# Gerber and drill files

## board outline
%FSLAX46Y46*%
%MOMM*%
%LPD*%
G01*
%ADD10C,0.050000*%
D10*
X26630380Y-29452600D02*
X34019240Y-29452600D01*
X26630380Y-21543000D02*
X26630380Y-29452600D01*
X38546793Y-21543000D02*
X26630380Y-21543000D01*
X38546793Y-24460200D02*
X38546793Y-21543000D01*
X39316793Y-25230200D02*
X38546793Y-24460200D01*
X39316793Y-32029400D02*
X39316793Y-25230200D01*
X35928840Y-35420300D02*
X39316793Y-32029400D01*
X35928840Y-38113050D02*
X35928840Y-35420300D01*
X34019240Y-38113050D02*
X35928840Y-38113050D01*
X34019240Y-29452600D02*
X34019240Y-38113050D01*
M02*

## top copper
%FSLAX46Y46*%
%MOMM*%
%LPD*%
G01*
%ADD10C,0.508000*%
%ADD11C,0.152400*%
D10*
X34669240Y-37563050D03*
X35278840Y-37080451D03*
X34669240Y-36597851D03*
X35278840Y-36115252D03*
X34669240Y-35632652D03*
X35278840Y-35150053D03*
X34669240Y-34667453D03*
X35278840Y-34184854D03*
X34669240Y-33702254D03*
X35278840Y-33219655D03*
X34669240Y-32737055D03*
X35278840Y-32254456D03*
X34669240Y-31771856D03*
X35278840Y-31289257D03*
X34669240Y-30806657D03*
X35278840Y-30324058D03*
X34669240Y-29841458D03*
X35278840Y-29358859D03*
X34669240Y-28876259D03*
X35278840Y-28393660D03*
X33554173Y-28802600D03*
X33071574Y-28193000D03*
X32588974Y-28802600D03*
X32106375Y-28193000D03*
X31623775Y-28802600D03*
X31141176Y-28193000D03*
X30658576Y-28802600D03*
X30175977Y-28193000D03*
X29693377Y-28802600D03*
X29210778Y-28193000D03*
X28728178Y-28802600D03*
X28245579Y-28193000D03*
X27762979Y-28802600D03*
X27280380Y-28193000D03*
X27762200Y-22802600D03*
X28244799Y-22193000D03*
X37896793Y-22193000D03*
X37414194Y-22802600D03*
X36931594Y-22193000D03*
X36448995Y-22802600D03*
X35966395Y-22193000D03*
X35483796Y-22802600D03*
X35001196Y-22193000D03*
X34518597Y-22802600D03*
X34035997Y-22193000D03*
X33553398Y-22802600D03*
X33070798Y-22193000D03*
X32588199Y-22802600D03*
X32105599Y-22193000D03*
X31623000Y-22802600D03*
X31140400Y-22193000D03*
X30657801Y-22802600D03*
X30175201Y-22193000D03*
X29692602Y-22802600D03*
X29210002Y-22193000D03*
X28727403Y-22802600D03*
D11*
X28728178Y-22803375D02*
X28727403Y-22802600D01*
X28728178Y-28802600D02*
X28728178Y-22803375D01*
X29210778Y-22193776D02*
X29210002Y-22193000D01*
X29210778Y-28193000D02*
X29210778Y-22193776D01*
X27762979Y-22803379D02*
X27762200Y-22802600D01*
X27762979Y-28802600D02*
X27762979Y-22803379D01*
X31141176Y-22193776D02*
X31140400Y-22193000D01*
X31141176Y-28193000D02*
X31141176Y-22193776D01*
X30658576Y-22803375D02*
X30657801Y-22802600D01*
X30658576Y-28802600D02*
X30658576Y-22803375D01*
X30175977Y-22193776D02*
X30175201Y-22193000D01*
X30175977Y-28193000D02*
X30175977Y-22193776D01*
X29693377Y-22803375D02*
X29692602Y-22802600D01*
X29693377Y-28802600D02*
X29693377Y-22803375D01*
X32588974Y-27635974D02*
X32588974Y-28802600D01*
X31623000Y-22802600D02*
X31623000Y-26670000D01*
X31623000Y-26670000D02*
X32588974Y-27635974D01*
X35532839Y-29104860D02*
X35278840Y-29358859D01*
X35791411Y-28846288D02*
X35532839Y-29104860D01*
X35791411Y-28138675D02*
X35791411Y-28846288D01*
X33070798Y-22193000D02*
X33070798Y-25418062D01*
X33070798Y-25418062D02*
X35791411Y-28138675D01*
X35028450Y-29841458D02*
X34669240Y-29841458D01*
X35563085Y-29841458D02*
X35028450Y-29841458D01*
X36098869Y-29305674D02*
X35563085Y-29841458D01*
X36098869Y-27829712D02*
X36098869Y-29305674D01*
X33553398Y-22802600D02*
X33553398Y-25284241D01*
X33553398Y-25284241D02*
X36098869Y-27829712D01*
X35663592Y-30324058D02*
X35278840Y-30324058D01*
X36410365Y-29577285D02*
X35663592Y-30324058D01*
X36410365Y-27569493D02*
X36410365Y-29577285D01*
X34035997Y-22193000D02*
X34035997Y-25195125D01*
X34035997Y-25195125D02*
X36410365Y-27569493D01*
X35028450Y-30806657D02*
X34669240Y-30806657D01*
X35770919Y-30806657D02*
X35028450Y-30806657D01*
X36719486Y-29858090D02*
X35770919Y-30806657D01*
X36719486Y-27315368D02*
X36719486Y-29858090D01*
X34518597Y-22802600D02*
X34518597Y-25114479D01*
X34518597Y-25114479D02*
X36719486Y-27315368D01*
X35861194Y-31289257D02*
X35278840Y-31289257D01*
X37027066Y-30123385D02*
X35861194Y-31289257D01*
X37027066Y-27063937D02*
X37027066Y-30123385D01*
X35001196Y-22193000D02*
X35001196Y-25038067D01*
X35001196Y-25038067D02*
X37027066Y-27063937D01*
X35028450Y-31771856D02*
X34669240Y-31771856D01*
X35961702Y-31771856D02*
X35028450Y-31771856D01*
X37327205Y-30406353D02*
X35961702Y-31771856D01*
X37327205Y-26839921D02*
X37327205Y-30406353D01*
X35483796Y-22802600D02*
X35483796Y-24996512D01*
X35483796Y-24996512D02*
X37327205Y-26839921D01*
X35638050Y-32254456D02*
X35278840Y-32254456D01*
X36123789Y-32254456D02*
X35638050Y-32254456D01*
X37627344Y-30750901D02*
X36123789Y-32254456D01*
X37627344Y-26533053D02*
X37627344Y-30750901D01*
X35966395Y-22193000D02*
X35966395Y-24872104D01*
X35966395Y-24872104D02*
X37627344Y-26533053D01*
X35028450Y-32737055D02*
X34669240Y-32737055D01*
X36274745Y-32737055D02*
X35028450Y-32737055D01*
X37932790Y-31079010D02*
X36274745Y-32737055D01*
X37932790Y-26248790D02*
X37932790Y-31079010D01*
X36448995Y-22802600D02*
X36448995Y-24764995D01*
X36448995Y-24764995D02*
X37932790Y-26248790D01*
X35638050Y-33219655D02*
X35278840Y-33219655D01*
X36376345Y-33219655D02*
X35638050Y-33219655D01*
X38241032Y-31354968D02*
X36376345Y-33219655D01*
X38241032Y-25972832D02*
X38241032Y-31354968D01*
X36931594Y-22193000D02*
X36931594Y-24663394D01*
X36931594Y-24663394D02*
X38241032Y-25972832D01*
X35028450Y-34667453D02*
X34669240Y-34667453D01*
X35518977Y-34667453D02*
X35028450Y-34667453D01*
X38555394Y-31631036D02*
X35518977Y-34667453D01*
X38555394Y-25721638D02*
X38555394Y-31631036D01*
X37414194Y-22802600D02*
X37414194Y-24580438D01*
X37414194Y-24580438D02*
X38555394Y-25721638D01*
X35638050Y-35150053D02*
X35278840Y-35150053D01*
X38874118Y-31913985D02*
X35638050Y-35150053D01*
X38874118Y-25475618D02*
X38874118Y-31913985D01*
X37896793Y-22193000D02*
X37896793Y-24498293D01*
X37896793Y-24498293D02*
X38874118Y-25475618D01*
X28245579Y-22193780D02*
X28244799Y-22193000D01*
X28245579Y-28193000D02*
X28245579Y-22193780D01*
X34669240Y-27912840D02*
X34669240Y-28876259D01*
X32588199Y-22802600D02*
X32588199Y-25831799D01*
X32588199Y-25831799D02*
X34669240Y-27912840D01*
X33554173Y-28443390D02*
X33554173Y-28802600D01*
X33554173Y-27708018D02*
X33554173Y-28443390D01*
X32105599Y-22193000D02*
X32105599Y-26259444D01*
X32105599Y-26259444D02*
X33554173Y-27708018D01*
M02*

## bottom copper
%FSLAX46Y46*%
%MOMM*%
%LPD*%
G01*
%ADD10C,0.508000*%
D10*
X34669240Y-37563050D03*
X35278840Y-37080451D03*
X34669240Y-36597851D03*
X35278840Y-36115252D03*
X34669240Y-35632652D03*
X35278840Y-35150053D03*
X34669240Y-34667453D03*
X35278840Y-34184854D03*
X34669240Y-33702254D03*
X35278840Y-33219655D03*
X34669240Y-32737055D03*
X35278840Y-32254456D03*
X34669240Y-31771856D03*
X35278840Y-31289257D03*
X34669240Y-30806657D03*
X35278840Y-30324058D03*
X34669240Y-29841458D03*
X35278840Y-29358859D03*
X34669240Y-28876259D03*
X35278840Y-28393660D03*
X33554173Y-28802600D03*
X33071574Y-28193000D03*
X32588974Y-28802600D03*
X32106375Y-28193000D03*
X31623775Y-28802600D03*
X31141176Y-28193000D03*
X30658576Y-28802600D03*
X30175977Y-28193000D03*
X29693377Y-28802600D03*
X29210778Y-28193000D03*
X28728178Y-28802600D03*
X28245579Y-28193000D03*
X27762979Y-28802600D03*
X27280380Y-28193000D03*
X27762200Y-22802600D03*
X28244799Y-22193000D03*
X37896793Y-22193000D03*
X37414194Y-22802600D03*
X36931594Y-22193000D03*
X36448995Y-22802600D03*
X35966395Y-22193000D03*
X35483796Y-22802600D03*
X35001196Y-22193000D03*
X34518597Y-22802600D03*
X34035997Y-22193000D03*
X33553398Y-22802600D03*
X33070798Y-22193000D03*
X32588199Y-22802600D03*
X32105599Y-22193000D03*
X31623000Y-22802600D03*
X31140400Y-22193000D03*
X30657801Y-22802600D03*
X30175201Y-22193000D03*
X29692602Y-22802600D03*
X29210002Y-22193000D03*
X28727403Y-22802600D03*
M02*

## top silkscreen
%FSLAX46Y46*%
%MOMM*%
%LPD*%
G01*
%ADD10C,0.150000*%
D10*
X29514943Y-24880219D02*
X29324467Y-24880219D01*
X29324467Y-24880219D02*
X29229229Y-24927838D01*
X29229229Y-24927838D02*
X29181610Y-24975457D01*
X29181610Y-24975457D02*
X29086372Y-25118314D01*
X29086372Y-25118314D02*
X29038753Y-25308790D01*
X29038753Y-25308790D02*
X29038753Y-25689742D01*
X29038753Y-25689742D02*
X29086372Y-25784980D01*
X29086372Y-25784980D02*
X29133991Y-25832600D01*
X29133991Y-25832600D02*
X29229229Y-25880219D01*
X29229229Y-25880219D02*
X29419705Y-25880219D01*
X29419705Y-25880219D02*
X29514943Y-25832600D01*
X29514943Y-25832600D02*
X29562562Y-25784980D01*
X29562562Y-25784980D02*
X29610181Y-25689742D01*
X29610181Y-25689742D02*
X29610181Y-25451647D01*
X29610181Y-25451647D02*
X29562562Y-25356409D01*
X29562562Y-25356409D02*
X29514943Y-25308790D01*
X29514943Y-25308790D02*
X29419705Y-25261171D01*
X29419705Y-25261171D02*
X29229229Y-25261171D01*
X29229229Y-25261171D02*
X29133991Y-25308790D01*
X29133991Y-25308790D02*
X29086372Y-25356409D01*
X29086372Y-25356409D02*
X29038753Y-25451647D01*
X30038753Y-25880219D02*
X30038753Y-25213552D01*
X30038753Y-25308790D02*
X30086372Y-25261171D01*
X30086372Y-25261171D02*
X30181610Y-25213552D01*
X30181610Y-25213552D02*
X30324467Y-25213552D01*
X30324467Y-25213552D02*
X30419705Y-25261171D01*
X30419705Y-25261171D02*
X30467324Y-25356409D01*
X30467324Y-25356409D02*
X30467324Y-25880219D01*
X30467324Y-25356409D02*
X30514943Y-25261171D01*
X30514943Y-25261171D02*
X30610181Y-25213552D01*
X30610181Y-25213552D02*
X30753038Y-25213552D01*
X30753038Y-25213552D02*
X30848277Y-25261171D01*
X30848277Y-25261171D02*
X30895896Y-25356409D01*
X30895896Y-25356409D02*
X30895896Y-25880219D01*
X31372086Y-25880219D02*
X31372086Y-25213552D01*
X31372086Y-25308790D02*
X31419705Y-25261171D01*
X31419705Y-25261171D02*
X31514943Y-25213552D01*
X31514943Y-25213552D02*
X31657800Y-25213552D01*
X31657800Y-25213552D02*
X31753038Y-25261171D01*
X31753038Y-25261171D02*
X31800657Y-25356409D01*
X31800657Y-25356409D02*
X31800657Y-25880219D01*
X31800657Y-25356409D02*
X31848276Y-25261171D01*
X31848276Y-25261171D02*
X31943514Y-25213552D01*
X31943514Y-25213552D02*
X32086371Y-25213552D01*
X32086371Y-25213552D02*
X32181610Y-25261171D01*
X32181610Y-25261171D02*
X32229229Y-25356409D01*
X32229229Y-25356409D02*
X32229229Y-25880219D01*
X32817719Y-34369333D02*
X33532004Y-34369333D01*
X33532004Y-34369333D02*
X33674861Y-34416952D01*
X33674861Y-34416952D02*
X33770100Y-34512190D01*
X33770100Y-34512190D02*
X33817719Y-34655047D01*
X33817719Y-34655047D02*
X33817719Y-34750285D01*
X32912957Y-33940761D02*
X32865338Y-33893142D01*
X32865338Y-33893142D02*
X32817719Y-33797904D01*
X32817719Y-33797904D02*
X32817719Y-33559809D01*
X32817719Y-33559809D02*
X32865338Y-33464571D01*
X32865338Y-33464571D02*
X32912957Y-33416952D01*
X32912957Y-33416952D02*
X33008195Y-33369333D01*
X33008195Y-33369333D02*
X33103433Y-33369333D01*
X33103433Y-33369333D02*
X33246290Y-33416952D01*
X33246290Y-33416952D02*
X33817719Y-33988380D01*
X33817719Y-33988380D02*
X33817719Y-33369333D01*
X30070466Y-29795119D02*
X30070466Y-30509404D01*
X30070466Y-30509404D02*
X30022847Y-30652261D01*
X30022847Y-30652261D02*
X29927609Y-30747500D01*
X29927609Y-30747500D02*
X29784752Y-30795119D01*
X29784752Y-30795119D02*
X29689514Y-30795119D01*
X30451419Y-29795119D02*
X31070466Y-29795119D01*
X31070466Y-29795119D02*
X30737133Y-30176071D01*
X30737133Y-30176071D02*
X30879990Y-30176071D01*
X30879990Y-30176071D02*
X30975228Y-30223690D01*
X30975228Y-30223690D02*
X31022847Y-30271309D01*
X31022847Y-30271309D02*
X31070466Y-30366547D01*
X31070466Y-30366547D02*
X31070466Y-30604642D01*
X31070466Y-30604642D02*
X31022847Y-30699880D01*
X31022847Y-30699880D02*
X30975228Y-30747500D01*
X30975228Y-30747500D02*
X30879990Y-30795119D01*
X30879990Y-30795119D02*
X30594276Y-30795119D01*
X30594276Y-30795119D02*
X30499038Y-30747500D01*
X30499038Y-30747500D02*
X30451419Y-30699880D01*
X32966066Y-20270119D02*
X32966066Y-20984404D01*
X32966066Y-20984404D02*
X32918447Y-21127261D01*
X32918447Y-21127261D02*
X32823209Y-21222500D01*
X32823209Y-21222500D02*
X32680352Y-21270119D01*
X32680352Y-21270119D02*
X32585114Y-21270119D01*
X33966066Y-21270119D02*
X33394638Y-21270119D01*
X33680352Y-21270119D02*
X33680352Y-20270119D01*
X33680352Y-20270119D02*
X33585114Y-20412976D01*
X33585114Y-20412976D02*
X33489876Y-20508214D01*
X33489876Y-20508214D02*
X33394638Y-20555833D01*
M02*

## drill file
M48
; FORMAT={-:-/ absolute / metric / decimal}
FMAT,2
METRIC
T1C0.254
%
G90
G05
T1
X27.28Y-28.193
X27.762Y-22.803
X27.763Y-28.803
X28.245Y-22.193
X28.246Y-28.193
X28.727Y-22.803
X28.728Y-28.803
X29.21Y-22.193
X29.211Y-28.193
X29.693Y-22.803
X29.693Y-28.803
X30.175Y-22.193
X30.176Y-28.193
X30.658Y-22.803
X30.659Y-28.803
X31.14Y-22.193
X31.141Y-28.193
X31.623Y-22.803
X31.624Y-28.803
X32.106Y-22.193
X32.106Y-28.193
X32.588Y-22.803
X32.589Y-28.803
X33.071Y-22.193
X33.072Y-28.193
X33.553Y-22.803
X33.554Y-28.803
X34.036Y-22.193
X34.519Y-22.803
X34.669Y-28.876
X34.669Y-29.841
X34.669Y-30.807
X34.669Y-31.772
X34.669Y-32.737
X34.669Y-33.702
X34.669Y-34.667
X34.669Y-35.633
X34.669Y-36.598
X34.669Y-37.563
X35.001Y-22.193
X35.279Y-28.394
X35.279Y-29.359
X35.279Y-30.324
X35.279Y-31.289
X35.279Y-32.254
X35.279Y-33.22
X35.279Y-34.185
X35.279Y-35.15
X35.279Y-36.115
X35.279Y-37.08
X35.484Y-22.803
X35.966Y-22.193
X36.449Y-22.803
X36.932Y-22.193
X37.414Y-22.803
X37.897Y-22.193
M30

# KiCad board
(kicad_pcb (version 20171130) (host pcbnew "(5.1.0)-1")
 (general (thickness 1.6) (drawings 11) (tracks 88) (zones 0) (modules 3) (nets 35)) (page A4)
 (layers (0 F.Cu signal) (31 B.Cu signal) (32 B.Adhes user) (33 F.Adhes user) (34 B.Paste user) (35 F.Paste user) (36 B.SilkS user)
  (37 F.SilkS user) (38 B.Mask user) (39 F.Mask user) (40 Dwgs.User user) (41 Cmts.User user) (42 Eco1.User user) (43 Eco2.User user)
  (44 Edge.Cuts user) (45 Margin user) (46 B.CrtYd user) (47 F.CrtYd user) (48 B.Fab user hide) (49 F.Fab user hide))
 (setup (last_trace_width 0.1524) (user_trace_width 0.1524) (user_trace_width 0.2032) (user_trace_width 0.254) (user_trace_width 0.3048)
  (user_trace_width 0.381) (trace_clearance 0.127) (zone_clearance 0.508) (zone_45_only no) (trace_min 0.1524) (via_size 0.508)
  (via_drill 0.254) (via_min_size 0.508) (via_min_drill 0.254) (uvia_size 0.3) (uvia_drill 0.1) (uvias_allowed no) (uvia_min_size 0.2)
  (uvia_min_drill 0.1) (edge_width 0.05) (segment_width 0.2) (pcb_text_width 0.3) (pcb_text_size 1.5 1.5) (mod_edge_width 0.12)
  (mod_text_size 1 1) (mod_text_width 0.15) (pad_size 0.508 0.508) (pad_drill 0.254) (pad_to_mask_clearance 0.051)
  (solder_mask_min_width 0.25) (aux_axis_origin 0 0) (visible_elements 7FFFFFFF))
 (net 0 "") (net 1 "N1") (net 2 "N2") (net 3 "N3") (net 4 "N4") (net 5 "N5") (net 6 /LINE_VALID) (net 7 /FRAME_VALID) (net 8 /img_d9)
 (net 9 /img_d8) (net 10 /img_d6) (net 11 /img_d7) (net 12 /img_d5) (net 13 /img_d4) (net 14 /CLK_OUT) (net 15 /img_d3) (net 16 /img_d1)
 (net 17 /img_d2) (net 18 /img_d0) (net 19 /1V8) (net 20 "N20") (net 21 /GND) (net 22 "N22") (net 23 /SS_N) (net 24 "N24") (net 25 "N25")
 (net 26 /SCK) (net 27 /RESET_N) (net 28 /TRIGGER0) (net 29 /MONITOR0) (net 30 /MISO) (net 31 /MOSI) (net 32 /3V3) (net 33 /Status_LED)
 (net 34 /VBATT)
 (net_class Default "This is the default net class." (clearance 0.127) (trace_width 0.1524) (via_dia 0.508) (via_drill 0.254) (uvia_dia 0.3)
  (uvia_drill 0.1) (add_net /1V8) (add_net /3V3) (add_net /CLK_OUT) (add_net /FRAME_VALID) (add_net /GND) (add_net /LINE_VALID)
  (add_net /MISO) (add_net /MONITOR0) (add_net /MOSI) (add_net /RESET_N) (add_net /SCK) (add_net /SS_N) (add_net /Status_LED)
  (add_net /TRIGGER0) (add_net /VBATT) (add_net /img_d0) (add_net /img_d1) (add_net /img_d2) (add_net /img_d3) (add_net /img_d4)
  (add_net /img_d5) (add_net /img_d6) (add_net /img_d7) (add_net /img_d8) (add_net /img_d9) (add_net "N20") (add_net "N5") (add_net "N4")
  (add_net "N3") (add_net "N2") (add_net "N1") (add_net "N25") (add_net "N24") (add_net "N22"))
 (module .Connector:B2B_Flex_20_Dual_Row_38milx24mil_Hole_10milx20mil (layer F.Cu) (at 35.27884 28.39366 270)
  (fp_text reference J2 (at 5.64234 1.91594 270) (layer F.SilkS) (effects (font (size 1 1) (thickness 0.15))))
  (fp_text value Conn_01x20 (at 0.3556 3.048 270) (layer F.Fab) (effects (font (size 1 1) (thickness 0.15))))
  (pad 20 thru_hole circle (at 9.16939 0.6096 270) (size 0.508 0.508) (drill 0.254) (layers *.Cu *.Mask) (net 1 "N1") (zone_connect 0))
  (pad 19 thru_hole circle (at 8.686791 0 270) (size 0.508 0.508) (drill 0.254) (layers *.Cu *.Mask) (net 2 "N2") (zone_connect 0))
  (pad 18 thru_hole circle (at 8.204191 0.6096 270) (size 0.508 0.508) (drill 0.254) (layers *.Cu *.Mask) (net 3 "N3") (zone_connect 0))
  (pad 17 thru_hole circle (at 7.721592 0 270) (size 0.508 0.508) (drill 0.254) (layers *.Cu *.Mask) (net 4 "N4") (zone_connect 0))
  (pad 16 thru_hole circle (at 7.238992 0.6096 270) (size 0.508 0.508) (drill 0.254) (layers *.Cu *.Mask) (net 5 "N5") (zone_connect 0))
  (pad 15 thru_hole circle (at 6.756393 0 270) (size 0.508 0.508) (drill 0.254) (layers *.Cu *.Mask) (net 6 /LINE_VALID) (zone_connect 0))
  (pad 14 thru_hole circle (at 6.273793 0.6096 270) (size 0.508 0.508) (drill 0.254) (layers *.Cu *.Mask) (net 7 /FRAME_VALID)
   (zone_connect 0))
  (pad 13 thru_hole circle (at 5.791194 0 270) (size 0.508 0.508) (drill 0.254) (layers *.Cu *.Mask) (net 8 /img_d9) (zone_connect 0))
  (pad 12 thru_hole circle (at 5.308594 0.6096 270) (size 0.508 0.508) (drill 0.254) (layers *.Cu *.Mask) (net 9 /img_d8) (zone_connect 0))
  (pad 11 thru_hole circle (at 4.825995 0 270) (size 0.508 0.508) (drill 0.254) (layers *.Cu *.Mask) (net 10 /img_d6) (zone_connect 0))
  (pad 10 thru_hole circle (at 4.343395 0.6096 270) (size 0.508 0.508) (drill 0.254) (layers *.Cu *.Mask) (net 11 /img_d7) (zone_connect 0))
  (pad 9 thru_hole circle (at 3.860796 0 270) (size 0.508 0.508) (drill 0.254) (layers *.Cu *.Mask) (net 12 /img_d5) (zone_connect 0))
  (pad 8 thru_hole circle (at 3.378196 0.6096 270) (size 0.508 0.508) (drill 0.254) (layers *.Cu *.Mask) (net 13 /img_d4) (zone_connect 0))
  (pad 7 thru_hole circle (at 2.895597 0 270) (size 0.508 0.508) (drill 0.254) (layers *.Cu *.Mask) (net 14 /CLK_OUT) (zone_connect 0))
  (pad 6 thru_hole circle (at 2.412997 0.6096 270) (size 0.508 0.508) (drill 0.254) (layers *.Cu *.Mask) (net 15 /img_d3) (zone_connect 0))
  (pad 5 thru_hole circle (at 1.930398 0 270) (size 0.508 0.508) (drill 0.254) (layers *.Cu *.Mask) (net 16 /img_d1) (zone_connect 0))
  (pad 4 thru_hole circle (at 1.447798 0.6096 270) (size 0.508 0.508) (drill 0.254) (layers *.Cu *.Mask) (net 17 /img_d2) (zone_connect 0))
  (pad 3 thru_hole circle (at 0.965199 0 270) (size 0.508 0.508) (drill 0.254) (layers *.Cu *.Mask) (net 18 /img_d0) (zone_connect 0))
  (pad 2 thru_hole circle (at 0.482599 0.6096 270) (size 0.508 0.508) (drill 0.254) (layers *.Cu *.Mask) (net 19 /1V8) (zone_connect 0))
  (pad 1 thru_hole circle (at 0 0 270) (size 0.508 0.508) (drill 0.254) (layers *.Cu *.Mask) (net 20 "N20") (zone_connect 0)))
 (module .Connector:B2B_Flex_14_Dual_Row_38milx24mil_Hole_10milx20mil (layer F.Cu) (at 27.28038 28.193)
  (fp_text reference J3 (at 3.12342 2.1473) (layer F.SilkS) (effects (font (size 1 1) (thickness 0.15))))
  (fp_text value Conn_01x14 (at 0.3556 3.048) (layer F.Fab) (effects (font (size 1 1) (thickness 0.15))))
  (pad 14 thru_hole circle (at 6.273793 0.6096) (size 0.508 0.508) (drill 0.254) (layers *.Cu *.Mask) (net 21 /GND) (zone_connect 0))
  (pad 13 thru_hole circle (at 5.791194 0) (size 0.508 0.508) (drill 0.254) (layers *.Cu *.Mask) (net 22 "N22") (zone_connect 0))
  (pad 12 thru_hole circle (at 5.308594 0.6096) (size 0.508 0.508) (drill 0.254) (layers *.Cu *.Mask) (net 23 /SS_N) (zone_connect 0))
  (pad 11 thru_hole circle (at 4.825995 0) (size 0.508 0.508) (drill 0.254) (layers *.Cu *.Mask) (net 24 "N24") (zone_connect 0))
  (pad 10 thru_hole circle (at 4.343395 0.6096) (size 0.508 0.508) (drill 0.254) (layers *.Cu *.Mask) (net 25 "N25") (zone_connect 0))
  (pad 9 thru_hole circle (at 3.860796 0) (size 0.508 0.508) (drill 0.254) (layers *.Cu *.Mask) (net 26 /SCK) (zone_connect 0))
  (pad 8 thru_hole circle (at 3.378196 0.6096) (size 0.508 0.508) (drill 0.254) (layers *.Cu *.Mask) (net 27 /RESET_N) (zone_connect 0))
  (pad 7 thru_hole circle (at 2.895597 0) (size 0.508 0.508) (drill 0.254) (layers *.Cu *.Mask) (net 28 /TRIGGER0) (zone_connect 0))
  (pad 6 thru_hole circle (at 2.412997 0.6096) (size 0.508 0.508) (drill 0.254) (layers *.Cu *.Mask) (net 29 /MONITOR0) (zone_connect 0))
  (pad 5 thru_hole circle (at 1.930398 0) (size 0.508 0.508) (drill 0.254) (layers *.Cu *.Mask) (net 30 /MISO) (zone_connect 0))
  (pad 4 thru_hole circle (at 1.447798 0.6096) (size 0.508 0.508) (drill 0.254) (layers *.Cu *.Mask) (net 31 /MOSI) (zone_connect 0))
  (pad 3 thru_hole circle (at 0.965199 0) (size 0.508 0.508) (drill 0.254) (layers *.Cu *.Mask) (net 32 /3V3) (zone_connect 0))
  (pad 2 thru_hole circle (at 0.482599 0.6096) (size 0.508 0.508) (drill 0.254) (layers *.Cu *.Mask) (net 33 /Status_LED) (zone_connect 0))
  (pad 1 thru_hole circle (at 0 0) (size 0.508 0.508) (drill 0.254) (layers *.Cu *.Mask) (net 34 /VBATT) (zone_connect 0)))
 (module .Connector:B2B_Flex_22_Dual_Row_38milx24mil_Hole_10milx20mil (layer F.Cu) (at 37.896793 22.193 180)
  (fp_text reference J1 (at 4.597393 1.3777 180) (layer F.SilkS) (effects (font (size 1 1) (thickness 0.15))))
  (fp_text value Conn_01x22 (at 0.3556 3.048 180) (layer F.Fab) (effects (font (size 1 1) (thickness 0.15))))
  (pad 22 thru_hole circle (at 10.134593 -0.6096 180) (size 0.508 0.508) (drill 0.254) (layers *.Cu *.Mask) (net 33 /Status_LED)
   (zone_connect 0))
  (pad 21 thru_hole circle (at 9.651994 0 180) (size 0.508 0.508) (drill 0.254) (layers *.Cu *.Mask) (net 32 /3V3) (zone_connect 0))
  (pad 1 thru_hole circle (at 0 0 180) (size 0.508 0.508) (drill 0.254) (layers *.Cu *.Mask) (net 6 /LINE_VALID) (zone_connect 0))
  (pad 2 thru_hole circle (at 0.482599 -0.6096 180) (size 0.508 0.508) (drill 0.254) (layers *.Cu *.Mask) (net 7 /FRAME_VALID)
   (zone_connect 0))
  (pad 3 thru_hole circle (at 0.965199 0 180) (size 0.508 0.508) (drill 0.254) (layers *.Cu *.Mask) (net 10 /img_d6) (zone_connect 0))
  (pad 4 thru_hole circle (at 1.447798 -0.6096 180) (size 0.508 0.508) (drill 0.254) (layers *.Cu *.Mask) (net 11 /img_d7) (zone_connect 0))
  (pad 5 thru_hole circle (at 1.930398 0 180) (size 0.508 0.508) (drill 0.254) (layers *.Cu *.Mask) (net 12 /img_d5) (zone_connect 0))
  (pad 6 thru_hole circle (at 2.412997 -0.6096 180) (size 0.508 0.508) (drill 0.254) (layers *.Cu *.Mask) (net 13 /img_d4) (zone_connect 0))
  (pad 7 thru_hole circle (at 2.895597 0 180) (size 0.508 0.508) (drill 0.254) (layers *.Cu *.Mask) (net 14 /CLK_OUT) (zone_connect 0))
  (pad 8 thru_hole circle (at 3.378196 -0.6096 180) (size 0.508 0.508) (drill 0.254) (layers *.Cu *.Mask) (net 15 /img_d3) (zone_connect 0))
  (pad 9 thru_hole circle (at 3.860796 0 180) (size 0.508 0.508) (drill 0.254) (layers *.Cu *.Mask) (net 16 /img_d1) (zone_connect 0))
  (pad 10 thru_hole circle (at 4.343395 -0.6096 180) (size 0.508 0.508) (drill 0.254) (layers *.Cu *.Mask) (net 17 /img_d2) (zone_connect 0))
  (pad 11 thru_hole circle (at 4.825995 0 180) (size 0.508 0.508) (drill 0.254) (layers *.Cu *.Mask) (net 18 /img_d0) (zone_connect 0))
  (pad 12 thru_hole circle (at 5.308594 -0.6096 180) (size 0.508 0.508) (drill 0.254) (layers *.Cu *.Mask) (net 19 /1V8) (zone_connect 0))
  (pad 13 thru_hole circle (at 5.791194 0 180) (size 0.508 0.508) (drill 0.254) (layers *.Cu *.Mask) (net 21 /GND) (zone_connect 0))
  (pad 14 thru_hole circle (at 6.273793 -0.6096 180) (size 0.508 0.508) (drill 0.254) (layers *.Cu *.Mask) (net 23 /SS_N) (zone_connect 0))
  (pad 15 thru_hole circle (at 6.756393 0 180) (size 0.508 0.508) (drill 0.254) (layers *.Cu *.Mask) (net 26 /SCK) (zone_connect 0))
  (pad 16 thru_hole circle (at 7.238992 -0.6096 180) (size 0.508 0.508) (drill 0.254) (layers *.Cu *.Mask) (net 27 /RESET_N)
   (zone_connect 0))
  (pad 17 thru_hole circle (at 7.721592 0 180) (size 0.508 0.508) (drill 0.254) (layers *.Cu *.Mask) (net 28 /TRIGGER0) (zone_connect 0))
  (pad 18 thru_hole circle (at 8.204191 -0.6096 180) (size 0.508 0.508) (drill 0.254) (layers *.Cu *.Mask) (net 29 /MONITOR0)
   (zone_connect 0))
  (pad 19 thru_hole circle (at 8.686791 0 180) (size 0.508 0.508) (drill 0.254) (layers *.Cu *.Mask) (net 30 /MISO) (zone_connect 0))
  (pad 20 thru_hole circle (at 9.16939 -0.6096 180) (size 0.508 0.508) (drill 0.254) (layers *.Cu *.Mask) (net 31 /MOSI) (zone_connect 0)))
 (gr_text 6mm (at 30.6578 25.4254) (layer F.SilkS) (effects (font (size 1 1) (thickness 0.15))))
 (gr_line (start 26.63038 29.4526) (end 34.01924 29.4526) (layer Edge.Cuts) (width 0.05))
 (gr_line (start 26.63038 21.543) (end 26.63038 29.4526) (layer Edge.Cuts) (width 0.05))
 (gr_line (start 38.546793 21.543) (end 26.63038 21.543) (layer Edge.Cuts) (width 0.05))
 (gr_line (start 38.546793 24.4602) (end 38.546793 21.543) (layer Edge.Cuts) (width 0.05))
 (gr_line (start 39.316793 25.2302) (end 38.546793 24.4602) (layer Edge.Cuts) (width 0.05))
 (gr_line (start 39.316793 32.0294) (end 39.316793 25.2302) (layer Edge.Cuts) (width 0.05))
 (gr_line (start 35.92884 35.4203) (end 39.316793 32.0294) (layer Edge.Cuts) (width 0.05))
 (gr_line (start 35.92884 38.11305) (end 35.92884 35.4203) (layer Edge.Cuts) (width 0.05))
 (gr_line (start 34.01924 38.11305) (end 35.92884 38.11305) (layer Edge.Cuts) (width 0.05))
 (gr_line (start 34.01924 29.4526) (end 34.01924 38.11305) (layer Edge.Cuts) (width 0.05))
 (segment (start 28.728178 22.803375) (end 28.727403 22.8026) (width 0.1524) (layer F.Cu) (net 31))
 (segment (start 28.728178 28.8026) (end 28.728178 22.803375) (width 0.1524) (layer F.Cu) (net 31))
 (segment (start 29.210778 22.193776) (end 29.210002 22.193) (width 0.1524) (layer F.Cu) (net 30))
 (segment (start 29.210778 28.193) (end 29.210778 22.193776) (width 0.1524) (layer F.Cu) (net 30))
 (segment (start 27.762979 22.803379) (end 27.7622 22.8026) (width 0.1524) (layer F.Cu) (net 33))
 (segment (start 27.762979 28.8026) (end 27.762979 22.803379) (width 0.1524) (layer F.Cu) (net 33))
 (segment (start 31.141176 22.193776) (end 31.1404 22.193) (width 0.1524) (layer F.Cu) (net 26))
 (segment (start 31.141176 28.193) (end 31.141176 22.193776) (width 0.1524) (layer F.Cu) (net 26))
 (segment (start 30.658576 22.803375) (end 30.657801 22.8026) (width 0.1524) (layer F.Cu) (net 27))
 (segment (start 30.658576 28.8026) (end 30.658576 22.803375) (width 0.1524) (layer F.Cu) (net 27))
 (segment (start 30.175977 22.193776) (end 30.175201 22.193) (width 0.1524) (layer F.Cu) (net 28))
 (segment (start 30.175977 28.193) (end 30.175977 22.193776) (width 0.1524) (layer F.Cu) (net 28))
 (segment (start 29.693377 22.803375) (end 29.692602 22.8026) (width 0.1524) (layer F.Cu) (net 29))
 (segment (start 29.693377 28.8026) (end 29.693377 22.803375) (width 0.1524) (layer F.Cu) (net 29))
 (segment (start 32.588974 27.635974) (end 32.588974 28.8026) (width 0.1524) (layer F.Cu) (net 23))
 (segment (start 31.623 22.8026) (end 31.623 26.67) (width 0.1524) (layer F.Cu) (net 23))
 (segment (start 31.623 26.67) (end 32.588974 27.635974) (width 0.1524) (layer F.Cu) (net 23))
 (segment (start 35.532839 29.10486) (end 35.27884 29.358859) (width 0.1524) (layer F.Cu) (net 18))
 (segment (start 35.791411 28.846288) (end 35.532839 29.10486) (width 0.1524) (layer F.Cu) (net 18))
 (segment (start 35.791411 28.138675) (end 35.791411 28.846288) (width 0.1524) (layer F.Cu) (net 18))
 (segment (start 33.070798 22.193) (end 33.070798 25.418062) (width 0.1524) (layer F.Cu) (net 18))
 (segment (start 33.070798 25.418062) (end 35.791411 28.138675) (width 0.1524) (layer F.Cu) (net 18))
 (segment (start 35.02845 29.841458) (end 34.66924 29.841458) (width 0.1524) (layer F.Cu) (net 17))
 (segment (start 35.563085 29.841458) (end 35.02845 29.841458) (width 0.1524) (layer F.Cu) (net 17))
 (segment (start 36.098869 29.305674) (end 35.563085 29.841458) (width 0.1524) (layer F.Cu) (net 17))
 (segment (start 36.098869 27.829712) (end 36.098869 29.305674) (width 0.1524) (layer F.Cu) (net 17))
 (segment (start 33.553398 22.8026) (end 33.553398 25.284241) (width 0.1524) (layer F.Cu) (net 17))
 (segment (start 33.553398 25.284241) (end 36.098869 27.829712) (width 0.1524) (layer F.Cu) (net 17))
 (segment (start 35.663592 30.324058) (end 35.27884 30.324058) (width 0.1524) (layer F.Cu) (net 16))
 (segment (start 36.410365 29.577285) (end 35.663592 30.324058) (width 0.1524) (layer F.Cu) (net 16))
 (segment (start 36.410365 27.569493) (end 36.410365 29.577285) (width 0.1524) (layer F.Cu) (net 16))
 (segment (start 34.035997 22.193) (end 34.035997 25.195125) (width 0.1524) (layer F.Cu) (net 16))
 (segment (start 34.035997 25.195125) (end 36.410365 27.569493) (width 0.1524) (layer F.Cu) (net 16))
 (segment (start 35.02845 30.806657) (end 34.66924 30.806657) (width 0.1524) (layer F.Cu) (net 15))
 (segment (start 35.770919 30.806657) (end 35.02845 30.806657) (width 0.1524) (layer F.Cu) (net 15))
 (segment (start 36.719486 29.85809) (end 35.770919 30.806657) (width 0.1524) (layer F.Cu) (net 15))
 (segment (start 36.719486 27.315368) (end 36.719486 29.85809) (width 0.1524) (layer F.Cu) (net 15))
 (segment (start 34.518597 22.8026) (end 34.518597 25.114479) (width 0.1524) (layer F.Cu) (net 15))
 (segment (start 34.518597 25.114479) (end 36.719486 27.315368) (width 0.1524) (layer F.Cu) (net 15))
 (segment (start 35.861194 31.289257) (end 35.27884 31.289257) (width 0.1524) (layer F.Cu) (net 14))
 (segment (start 37.027066 30.123385) (end 35.861194 31.289257) (width 0.1524) (layer F.Cu) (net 14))
 (segment (start 37.027066 27.063937) (end 37.027066 30.123385) (width 0.1524) (layer F.Cu) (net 14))
 (segment (start 35.001196 22.193) (end 35.001196 25.038067) (width 0.1524) (layer F.Cu) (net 14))
 (segment (start 35.001196 25.038067) (end 37.027066 27.063937) (width 0.1524) (layer F.Cu) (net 14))
 (segment (start 35.02845 31.771856) (end 34.66924 31.771856) (width 0.1524) (layer F.Cu) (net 13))
 (segment (start 35.961702 31.771856) (end 35.02845 31.771856) (width 0.1524) (layer F.Cu) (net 13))
 (segment (start 37.327205 30.406353) (end 35.961702 31.771856) (width 0.1524) (layer F.Cu) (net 13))
 (segment (start 37.327205 26.839921) (end 37.327205 30.406353) (width 0.1524) (layer F.Cu) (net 13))
 (segment (start 35.483796 22.8026) (end 35.483796 24.996512) (width 0.1524) (layer F.Cu) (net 13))
 (segment (start 35.483796 24.996512) (end 37.327205 26.839921) (width 0.1524) (layer F.Cu) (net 13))
 (segment (start 35.63805 32.254456) (end 35.27884 32.254456) (width 0.1524) (layer F.Cu) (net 12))
 (segment (start 36.123789 32.254456) (end 35.63805 32.254456) (width 0.1524) (layer F.Cu) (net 12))
 (segment (start 37.627344 30.750901) (end 36.123789 32.254456) (width 0.1524) (layer F.Cu) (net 12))
 (segment (start 37.627344 26.533053) (end 37.627344 30.750901) (width 0.1524) (layer F.Cu) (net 12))
 (segment (start 35.966395 22.193) (end 35.966395 24.872104) (width 0.1524) (layer F.Cu) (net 12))
 (segment (start 35.966395 24.872104) (end 37.627344 26.533053) (width 0.1524) (layer F.Cu) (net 12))
 (segment (start 35.02845 32.737055) (end 34.66924 32.737055) (width 0.1524) (layer F.Cu) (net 11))
 (segment (start 36.274745 32.737055) (end 35.02845 32.737055) (width 0.1524) (layer F.Cu) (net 11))
 (segment (start 37.93279 31.07901) (end 36.274745 32.737055) (width 0.1524) (layer F.Cu) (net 11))
 (segment (start 37.93279 26.24879) (end 37.93279 31.07901) (width 0.1524) (layer F.Cu) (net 11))
 (segment (start 36.448995 22.8026) (end 36.448995 24.764995) (width 0.1524) (layer F.Cu) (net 11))
 (segment (start 36.448995 24.764995) (end 37.93279 26.24879) (width 0.1524) (layer F.Cu) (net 11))
 (segment (start 35.63805 33.219655) (end 35.27884 33.219655) (width 0.1524) (layer F.Cu) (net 10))
 (segment (start 36.376345 33.219655) (end 35.63805 33.219655) (width 0.1524) (layer F.Cu) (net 10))
 (segment (start 38.241032 31.354968) (end 36.376345 33.219655) (width 0.1524) (layer F.Cu) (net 10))
 (segment (start 38.241032 25.972832) (end 38.241032 31.354968) (width 0.1524) (layer F.Cu) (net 10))
 (segment (start 36.931594 22.193) (end 36.931594 24.663394) (width 0.1524) (layer F.Cu) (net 10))
 (segment (start 36.931594 24.663394) (end 38.241032 25.972832) (width 0.1524) (layer F.Cu) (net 10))
 (segment (start 35.02845 34.667453) (end 34.66924 34.667453) (width 0.1524) (layer F.Cu) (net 7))
 (segment (start 35.518977 34.667453) (end 35.02845 34.667453) (width 0.1524) (layer F.Cu) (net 7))
 (segment (start 38.555394 31.631036) (end 35.518977 34.667453) (width 0.1524) (layer F.Cu) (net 7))
 (segment (start 38.555394 25.721638) (end 38.555394 31.631036) (width 0.1524) (layer F.Cu) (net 7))
 (segment (start 37.414194 22.8026) (end 37.414194 24.580438) (width 0.1524) (layer F.Cu) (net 7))
 (segment (start 37.414194 24.580438) (end 38.555394 25.721638) (width 0.1524) (layer F.Cu) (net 7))
 (segment (start 35.63805 35.150053) (end 35.27884 35.150053) (width 0.1524) (layer F.Cu) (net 6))
 (segment (start 38.874118 31.913985) (end 35.63805 35.150053) (width 0.1524) (layer F.Cu) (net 6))
 (segment (start 38.874118 25.475618) (end 38.874118 31.913985) (width 0.1524) (layer F.Cu) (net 6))
 (segment (start 37.896793 22.193) (end 37.896793 24.498293) (width 0.1524) (layer F.Cu) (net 6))
 (segment (start 37.896793 24.498293) (end 38.874118 25.475618) (width 0.1524) (layer F.Cu) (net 6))
 (segment (start 28.245579 22.19378) (end 28.244799 22.193) (width 0.1524) (layer F.Cu) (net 32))
 (segment (start 28.245579 28.193) (end 28.245579 22.19378) (width 0.1524) (layer F.Cu) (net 32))
 (segment (start 34.66924 27.91284) (end 34.66924 28.876259) (width 0.1524) (layer F.Cu) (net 19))
 (segment (start 32.588199 22.8026) (end 32.588199 25.831799) (width 0.1524) (layer F.Cu) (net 19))
 (segment (start 32.588199 25.831799) (end 34.66924 27.91284) (width 0.1524) (layer F.Cu) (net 19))
 (segment (start 33.554173 28.44339) (end 33.554173 28.8026) (width 0.1524) (layer F.Cu) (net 21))
 (segment (start 33.554173 27.708018) (end 33.554173 28.44339) (width 0.1524) (layer F.Cu) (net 21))
 (segment (start 32.105599 22.193) (end 32.105599 26.259444) (width 0.1524) (layer F.Cu) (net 21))
 (segment (start 32.105599 26.259444) (end 33.554173 27.708018) (width 0.1524) (layer F.Cu) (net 21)))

